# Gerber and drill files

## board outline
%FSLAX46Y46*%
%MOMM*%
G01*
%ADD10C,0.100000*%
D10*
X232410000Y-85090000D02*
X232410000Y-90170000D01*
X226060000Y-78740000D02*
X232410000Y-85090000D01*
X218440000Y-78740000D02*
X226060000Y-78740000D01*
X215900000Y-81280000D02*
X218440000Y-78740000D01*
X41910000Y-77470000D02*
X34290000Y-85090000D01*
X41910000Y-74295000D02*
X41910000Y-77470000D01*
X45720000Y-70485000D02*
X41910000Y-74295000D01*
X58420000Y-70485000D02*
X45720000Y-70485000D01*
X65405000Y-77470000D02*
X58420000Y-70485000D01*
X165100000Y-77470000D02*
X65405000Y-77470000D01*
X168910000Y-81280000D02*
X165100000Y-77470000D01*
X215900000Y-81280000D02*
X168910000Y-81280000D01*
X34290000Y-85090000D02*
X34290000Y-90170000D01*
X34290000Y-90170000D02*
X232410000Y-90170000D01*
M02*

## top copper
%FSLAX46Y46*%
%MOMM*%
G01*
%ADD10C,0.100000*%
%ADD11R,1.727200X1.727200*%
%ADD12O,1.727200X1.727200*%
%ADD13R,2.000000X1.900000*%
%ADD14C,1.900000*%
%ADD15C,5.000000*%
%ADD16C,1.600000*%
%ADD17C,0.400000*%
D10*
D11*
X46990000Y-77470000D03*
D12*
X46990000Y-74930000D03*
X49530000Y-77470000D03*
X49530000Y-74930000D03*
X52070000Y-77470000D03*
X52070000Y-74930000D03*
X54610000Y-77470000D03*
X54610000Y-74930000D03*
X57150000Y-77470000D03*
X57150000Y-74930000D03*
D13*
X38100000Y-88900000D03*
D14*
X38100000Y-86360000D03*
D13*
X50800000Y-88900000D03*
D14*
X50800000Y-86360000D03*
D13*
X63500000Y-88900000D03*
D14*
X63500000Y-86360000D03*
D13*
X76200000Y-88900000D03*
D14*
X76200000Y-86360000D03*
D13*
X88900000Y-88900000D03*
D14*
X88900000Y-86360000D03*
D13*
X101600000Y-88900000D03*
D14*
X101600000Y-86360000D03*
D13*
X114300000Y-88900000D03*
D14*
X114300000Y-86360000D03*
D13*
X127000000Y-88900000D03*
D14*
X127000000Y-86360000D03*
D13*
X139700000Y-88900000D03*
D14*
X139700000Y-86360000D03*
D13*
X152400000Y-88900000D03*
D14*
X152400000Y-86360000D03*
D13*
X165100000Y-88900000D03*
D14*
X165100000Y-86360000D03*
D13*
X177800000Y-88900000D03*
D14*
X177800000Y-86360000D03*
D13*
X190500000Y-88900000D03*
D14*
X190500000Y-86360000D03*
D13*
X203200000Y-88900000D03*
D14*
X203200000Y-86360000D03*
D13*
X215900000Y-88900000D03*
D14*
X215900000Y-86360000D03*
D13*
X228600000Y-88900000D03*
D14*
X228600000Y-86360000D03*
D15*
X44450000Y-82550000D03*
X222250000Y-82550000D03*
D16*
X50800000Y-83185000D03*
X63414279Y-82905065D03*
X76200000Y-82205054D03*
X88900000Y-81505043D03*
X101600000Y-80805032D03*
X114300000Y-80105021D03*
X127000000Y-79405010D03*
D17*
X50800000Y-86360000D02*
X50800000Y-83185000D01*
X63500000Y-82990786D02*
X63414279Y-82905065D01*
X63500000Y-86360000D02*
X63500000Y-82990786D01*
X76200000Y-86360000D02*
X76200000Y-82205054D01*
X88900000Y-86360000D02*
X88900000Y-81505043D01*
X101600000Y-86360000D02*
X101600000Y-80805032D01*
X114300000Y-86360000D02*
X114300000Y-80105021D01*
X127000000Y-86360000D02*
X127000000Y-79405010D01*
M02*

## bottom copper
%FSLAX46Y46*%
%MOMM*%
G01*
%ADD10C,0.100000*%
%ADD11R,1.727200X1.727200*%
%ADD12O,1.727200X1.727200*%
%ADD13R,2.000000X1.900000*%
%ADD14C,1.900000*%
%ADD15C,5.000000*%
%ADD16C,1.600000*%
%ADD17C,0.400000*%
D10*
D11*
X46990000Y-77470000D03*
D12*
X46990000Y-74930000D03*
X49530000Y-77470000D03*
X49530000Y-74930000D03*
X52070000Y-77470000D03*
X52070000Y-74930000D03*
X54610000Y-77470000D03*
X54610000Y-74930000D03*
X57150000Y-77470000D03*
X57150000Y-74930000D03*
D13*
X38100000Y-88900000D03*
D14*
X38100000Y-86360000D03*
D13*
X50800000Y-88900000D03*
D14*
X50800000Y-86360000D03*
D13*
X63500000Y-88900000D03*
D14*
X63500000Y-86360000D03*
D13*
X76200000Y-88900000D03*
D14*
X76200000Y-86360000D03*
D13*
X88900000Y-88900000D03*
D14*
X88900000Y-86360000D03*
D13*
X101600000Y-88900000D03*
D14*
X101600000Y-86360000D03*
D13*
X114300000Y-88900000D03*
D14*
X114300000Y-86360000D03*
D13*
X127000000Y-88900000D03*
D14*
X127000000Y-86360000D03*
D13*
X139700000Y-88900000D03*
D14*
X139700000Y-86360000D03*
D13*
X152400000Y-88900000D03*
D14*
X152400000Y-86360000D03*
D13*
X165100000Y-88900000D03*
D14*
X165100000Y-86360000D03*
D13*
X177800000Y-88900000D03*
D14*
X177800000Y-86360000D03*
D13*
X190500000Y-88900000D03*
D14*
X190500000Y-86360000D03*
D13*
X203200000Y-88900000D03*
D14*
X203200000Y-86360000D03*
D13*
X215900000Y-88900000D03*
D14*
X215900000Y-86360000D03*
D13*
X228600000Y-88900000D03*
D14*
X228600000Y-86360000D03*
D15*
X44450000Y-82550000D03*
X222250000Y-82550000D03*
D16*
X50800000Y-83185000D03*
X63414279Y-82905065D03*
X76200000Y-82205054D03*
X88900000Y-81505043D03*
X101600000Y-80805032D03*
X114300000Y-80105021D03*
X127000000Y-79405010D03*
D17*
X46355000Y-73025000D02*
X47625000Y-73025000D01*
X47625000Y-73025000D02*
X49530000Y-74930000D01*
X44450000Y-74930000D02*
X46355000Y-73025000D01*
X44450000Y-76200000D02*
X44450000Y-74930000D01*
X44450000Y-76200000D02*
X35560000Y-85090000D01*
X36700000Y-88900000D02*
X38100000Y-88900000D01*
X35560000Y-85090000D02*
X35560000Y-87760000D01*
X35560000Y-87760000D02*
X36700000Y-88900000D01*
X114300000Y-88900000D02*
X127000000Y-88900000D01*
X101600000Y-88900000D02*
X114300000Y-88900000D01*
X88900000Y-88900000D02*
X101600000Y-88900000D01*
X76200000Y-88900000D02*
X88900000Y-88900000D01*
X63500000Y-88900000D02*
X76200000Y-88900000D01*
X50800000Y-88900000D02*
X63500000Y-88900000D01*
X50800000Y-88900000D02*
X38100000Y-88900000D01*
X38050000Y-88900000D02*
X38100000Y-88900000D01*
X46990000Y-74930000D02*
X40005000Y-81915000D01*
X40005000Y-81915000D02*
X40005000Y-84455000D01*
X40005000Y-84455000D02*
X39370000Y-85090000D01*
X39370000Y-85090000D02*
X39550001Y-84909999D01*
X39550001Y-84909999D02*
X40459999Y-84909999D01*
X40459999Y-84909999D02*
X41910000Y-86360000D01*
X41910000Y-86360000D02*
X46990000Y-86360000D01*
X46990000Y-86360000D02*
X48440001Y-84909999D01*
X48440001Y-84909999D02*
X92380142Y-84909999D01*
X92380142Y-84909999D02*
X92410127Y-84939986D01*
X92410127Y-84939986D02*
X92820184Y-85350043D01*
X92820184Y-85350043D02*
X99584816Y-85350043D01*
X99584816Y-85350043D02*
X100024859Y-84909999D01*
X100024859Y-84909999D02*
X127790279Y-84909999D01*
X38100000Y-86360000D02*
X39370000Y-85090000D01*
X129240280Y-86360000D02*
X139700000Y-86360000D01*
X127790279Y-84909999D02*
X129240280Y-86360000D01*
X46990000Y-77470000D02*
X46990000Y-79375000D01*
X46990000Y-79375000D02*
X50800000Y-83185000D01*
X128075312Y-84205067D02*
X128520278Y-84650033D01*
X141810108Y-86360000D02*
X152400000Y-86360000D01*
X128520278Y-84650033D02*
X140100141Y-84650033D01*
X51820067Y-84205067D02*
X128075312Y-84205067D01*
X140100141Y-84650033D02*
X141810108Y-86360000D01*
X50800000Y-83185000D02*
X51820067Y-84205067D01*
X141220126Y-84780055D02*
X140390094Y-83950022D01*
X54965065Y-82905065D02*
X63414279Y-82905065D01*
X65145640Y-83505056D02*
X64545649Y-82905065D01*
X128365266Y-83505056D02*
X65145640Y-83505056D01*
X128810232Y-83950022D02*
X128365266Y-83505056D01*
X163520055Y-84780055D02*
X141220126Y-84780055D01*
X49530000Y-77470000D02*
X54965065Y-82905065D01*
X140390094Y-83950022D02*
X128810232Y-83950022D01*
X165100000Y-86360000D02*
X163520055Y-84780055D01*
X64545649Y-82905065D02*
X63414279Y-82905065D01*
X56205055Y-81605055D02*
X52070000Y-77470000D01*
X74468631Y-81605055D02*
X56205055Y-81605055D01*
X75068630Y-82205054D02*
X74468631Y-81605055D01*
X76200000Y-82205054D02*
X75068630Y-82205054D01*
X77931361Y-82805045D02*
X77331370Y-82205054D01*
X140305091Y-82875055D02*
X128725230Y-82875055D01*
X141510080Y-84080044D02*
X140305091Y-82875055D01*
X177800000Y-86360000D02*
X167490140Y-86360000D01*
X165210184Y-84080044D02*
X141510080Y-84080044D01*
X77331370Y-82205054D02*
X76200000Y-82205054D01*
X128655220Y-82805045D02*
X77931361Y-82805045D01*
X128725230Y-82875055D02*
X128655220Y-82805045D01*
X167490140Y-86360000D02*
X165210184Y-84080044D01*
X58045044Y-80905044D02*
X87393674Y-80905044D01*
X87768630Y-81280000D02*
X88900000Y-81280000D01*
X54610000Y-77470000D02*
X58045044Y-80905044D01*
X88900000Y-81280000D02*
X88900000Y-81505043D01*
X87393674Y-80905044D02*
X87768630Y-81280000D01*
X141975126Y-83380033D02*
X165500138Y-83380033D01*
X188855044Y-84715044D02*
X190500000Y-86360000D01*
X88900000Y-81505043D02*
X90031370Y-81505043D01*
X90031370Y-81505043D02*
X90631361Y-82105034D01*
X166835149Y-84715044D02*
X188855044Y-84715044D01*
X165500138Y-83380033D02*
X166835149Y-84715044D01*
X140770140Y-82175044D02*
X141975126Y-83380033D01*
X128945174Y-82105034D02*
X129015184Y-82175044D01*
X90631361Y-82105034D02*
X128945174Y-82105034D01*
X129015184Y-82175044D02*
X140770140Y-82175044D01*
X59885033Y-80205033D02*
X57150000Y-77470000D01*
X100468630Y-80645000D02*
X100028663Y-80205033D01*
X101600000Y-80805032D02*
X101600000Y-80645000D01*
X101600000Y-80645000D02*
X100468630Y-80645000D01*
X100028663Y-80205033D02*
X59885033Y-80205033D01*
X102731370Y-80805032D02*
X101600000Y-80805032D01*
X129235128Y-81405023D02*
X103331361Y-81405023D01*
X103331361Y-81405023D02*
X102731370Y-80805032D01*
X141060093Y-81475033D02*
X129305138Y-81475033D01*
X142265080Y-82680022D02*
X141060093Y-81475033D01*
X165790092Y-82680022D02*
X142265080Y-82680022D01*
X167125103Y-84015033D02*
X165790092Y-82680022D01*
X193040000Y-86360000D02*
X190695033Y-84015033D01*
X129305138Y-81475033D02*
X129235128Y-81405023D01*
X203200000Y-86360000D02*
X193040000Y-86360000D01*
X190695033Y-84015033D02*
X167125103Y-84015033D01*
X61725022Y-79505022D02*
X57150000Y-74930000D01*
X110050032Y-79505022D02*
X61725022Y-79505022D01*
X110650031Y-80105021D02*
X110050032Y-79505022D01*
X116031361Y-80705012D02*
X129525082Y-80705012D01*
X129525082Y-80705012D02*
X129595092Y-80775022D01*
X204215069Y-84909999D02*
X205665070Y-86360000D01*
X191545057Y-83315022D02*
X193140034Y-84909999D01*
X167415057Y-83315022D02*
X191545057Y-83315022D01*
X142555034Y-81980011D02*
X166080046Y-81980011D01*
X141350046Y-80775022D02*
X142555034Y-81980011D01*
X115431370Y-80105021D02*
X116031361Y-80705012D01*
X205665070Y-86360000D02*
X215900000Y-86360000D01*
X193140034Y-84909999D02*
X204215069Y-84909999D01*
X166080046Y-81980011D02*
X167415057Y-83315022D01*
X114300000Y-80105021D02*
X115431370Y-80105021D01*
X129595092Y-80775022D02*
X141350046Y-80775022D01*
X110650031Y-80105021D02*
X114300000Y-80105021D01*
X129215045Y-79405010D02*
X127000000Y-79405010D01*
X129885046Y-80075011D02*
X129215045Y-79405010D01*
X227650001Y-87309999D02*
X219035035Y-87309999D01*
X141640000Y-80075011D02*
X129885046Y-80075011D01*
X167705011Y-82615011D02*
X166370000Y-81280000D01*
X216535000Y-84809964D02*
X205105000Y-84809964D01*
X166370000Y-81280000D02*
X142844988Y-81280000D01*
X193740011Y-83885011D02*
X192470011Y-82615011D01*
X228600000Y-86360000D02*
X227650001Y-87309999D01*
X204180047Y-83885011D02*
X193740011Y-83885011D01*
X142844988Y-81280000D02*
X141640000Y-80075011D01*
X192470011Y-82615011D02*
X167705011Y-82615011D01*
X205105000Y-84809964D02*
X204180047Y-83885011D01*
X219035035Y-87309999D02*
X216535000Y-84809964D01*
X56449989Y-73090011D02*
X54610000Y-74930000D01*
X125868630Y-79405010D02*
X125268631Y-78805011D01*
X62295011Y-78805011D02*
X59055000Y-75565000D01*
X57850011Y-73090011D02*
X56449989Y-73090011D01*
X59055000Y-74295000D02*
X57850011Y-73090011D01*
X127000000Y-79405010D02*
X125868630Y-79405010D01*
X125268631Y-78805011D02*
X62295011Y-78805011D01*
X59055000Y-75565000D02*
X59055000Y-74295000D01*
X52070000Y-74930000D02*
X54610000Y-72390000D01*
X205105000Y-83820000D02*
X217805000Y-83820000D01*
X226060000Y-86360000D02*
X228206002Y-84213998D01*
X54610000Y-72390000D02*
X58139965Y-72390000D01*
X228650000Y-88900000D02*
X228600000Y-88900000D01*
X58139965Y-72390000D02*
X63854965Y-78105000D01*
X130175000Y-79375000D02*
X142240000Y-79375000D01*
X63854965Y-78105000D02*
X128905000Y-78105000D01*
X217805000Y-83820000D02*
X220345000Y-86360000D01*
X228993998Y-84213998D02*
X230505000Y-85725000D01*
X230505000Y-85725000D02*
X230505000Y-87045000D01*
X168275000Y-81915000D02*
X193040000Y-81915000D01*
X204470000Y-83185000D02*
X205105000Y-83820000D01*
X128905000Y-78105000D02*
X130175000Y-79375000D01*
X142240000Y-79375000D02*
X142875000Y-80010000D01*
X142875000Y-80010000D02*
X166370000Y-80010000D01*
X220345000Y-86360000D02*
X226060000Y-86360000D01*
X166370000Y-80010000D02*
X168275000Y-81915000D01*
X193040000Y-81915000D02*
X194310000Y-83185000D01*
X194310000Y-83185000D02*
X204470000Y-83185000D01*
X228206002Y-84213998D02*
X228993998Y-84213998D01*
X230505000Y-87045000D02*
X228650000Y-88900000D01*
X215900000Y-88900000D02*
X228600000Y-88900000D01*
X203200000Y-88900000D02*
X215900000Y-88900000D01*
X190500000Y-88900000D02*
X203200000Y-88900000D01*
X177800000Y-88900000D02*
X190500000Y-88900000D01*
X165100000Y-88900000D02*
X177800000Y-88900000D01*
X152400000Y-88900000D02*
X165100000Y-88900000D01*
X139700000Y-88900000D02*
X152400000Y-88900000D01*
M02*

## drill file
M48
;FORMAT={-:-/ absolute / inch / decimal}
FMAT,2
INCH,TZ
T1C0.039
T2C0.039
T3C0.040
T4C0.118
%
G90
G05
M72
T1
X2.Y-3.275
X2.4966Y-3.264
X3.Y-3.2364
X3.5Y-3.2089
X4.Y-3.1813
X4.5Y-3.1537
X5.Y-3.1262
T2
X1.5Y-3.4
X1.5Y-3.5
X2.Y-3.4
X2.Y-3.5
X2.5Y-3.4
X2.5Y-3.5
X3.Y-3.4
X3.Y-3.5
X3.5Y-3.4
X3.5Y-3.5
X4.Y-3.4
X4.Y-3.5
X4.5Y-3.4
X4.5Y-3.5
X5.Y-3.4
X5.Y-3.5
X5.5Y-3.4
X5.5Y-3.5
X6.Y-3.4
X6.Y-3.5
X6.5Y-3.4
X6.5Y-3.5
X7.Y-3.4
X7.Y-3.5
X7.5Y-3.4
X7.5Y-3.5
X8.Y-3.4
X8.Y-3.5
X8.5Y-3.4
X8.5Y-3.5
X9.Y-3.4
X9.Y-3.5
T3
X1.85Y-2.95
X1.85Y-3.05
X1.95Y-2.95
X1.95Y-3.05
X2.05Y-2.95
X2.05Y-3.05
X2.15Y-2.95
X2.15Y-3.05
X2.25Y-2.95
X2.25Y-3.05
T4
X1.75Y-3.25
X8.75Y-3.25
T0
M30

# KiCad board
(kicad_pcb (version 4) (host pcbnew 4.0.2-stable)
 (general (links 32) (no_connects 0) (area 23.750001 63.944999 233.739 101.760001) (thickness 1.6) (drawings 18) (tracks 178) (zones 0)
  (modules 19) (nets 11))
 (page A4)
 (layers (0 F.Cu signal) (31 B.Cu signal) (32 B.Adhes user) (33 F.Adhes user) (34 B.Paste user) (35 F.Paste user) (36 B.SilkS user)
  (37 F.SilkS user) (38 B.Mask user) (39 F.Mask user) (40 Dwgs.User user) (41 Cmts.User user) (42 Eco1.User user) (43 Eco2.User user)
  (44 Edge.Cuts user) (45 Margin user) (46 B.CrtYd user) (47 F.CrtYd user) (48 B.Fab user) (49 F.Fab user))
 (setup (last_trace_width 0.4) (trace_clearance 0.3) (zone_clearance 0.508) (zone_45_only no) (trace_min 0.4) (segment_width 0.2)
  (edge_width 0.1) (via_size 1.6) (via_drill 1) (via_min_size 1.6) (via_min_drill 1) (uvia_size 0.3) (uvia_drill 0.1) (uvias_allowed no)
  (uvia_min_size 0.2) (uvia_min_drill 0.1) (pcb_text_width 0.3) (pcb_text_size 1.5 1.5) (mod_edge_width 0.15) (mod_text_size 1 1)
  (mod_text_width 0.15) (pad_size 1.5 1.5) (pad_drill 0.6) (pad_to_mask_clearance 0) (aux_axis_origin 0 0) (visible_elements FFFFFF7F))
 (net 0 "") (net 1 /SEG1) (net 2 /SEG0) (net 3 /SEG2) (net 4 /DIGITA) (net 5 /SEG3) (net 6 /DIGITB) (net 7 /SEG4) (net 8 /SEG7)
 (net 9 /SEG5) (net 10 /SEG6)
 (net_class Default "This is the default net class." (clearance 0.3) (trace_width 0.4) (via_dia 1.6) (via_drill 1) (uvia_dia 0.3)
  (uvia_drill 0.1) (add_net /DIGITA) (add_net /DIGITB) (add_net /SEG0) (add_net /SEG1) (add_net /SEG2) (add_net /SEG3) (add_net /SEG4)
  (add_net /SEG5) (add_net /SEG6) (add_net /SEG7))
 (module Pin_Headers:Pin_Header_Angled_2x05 (layer F.Cu) (at 46.99 77.47 90)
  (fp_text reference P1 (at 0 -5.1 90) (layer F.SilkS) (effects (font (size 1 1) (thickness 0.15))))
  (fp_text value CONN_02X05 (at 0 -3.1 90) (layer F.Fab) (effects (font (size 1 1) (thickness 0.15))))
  (pad 1 thru_hole rect (at 0 0 90) (size 1.7272 1.7272) (drill 1.016) (layers *.Cu *.Mask F.SilkS) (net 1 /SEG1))
  (pad 2 thru_hole oval (at 2.54 0 90) (size 1.7272 1.7272) (drill 1.016) (layers *.Cu *.Mask F.SilkS) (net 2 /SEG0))
  (pad 3 thru_hole oval (at 0 2.54 90) (size 1.7272 1.7272) (drill 1.016) (layers *.Cu *.Mask F.SilkS) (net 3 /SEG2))
  (pad 4 thru_hole oval (at 2.54 2.54 90) (size 1.7272 1.7272) (drill 1.016) (layers *.Cu *.Mask F.SilkS) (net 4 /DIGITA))
  (pad 5 thru_hole oval (at 0 5.08 90) (size 1.7272 1.7272) (drill 1.016) (layers *.Cu *.Mask F.SilkS) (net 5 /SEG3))
  (pad 6 thru_hole oval (at 2.54 5.08 90) (size 1.7272 1.7272) (drill 1.016) (layers *.Cu *.Mask F.SilkS) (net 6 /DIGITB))
  (pad 7 thru_hole oval (at 0 7.62 90) (size 1.7272 1.7272) (drill 1.016) (layers *.Cu *.Mask F.SilkS) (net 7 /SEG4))
  (pad 8 thru_hole oval (at 2.54 7.62 90) (size 1.7272 1.7272) (drill 1.016) (layers *.Cu *.Mask F.SilkS) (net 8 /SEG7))
  (pad 9 thru_hole oval (at 0 10.16 90) (size 1.7272 1.7272) (drill 1.016) (layers *.Cu *.Mask F.SilkS) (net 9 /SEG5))
  (pad 10 thru_hole oval (at 2.54 10.16 90) (size 1.7272 1.7272) (drill 1.016) (layers *.Cu *.Mask F.SilkS) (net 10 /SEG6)))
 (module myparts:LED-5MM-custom (layer F.Cu) (at 38.1 88.9 90)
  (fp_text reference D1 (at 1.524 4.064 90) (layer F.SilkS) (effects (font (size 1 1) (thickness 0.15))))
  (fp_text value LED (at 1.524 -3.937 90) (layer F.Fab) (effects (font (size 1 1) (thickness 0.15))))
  (pad 1 thru_hole rect (at 0 0 180) (size 2 1.9) (drill 1.00076) (layers *.Cu *.Mask F.SilkS) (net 4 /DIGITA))
  (pad 2 thru_hole circle (at 2.54 0 90) (size 1.9 1.9) (drill 1.00076) (layers *.Cu *.Mask F.SilkS) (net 2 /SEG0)))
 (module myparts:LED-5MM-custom (layer F.Cu) (at 50.8 88.9 90)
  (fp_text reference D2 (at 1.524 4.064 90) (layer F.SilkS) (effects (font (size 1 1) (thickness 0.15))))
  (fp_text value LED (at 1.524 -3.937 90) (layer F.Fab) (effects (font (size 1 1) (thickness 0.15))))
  (pad 1 thru_hole rect (at 0 0 180) (size 2 1.9) (drill 1.00076) (layers *.Cu *.Mask F.SilkS) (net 4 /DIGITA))
  (pad 2 thru_hole circle (at 2.54 0 90) (size 1.9 1.9) (drill 1.00076) (layers *.Cu *.Mask F.SilkS) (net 1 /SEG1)))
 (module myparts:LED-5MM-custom (layer F.Cu) (at 63.5 88.9 90)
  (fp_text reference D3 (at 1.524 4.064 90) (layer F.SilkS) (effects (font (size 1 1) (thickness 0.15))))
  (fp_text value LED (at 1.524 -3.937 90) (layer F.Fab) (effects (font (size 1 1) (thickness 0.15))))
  (pad 1 thru_hole rect (at 0 0 180) (size 2 1.9) (drill 1.00076) (layers *.Cu *.Mask F.SilkS) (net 4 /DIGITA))
  (pad 2 thru_hole circle (at 2.54 0 90) (size 1.9 1.9) (drill 1.00076) (layers *.Cu *.Mask F.SilkS) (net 3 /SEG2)))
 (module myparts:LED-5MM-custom (layer F.Cu) (at 76.2 88.9 90)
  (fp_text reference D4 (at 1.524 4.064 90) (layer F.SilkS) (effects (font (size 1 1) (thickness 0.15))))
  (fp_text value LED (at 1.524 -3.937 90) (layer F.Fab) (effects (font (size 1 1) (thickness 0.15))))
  (pad 1 thru_hole rect (at 0 0 180) (size 2 1.9) (drill 1.00076) (layers *.Cu *.Mask F.SilkS) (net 4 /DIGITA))
  (pad 2 thru_hole circle (at 2.54 0 90) (size 1.9 1.9) (drill 1.00076) (layers *.Cu *.Mask F.SilkS) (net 5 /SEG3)))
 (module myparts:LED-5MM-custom (layer F.Cu) (at 88.9 88.9 90)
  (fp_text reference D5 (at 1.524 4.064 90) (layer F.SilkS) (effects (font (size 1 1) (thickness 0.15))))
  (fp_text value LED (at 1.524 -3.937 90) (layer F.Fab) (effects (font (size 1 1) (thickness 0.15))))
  (pad 1 thru_hole rect (at 0 0 180) (size 2 1.9) (drill 1.00076) (layers *.Cu *.Mask F.SilkS) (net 4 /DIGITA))
  (pad 2 thru_hole circle (at 2.54 0 90) (size 1.9 1.9) (drill 1.00076) (layers *.Cu *.Mask F.SilkS) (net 7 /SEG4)))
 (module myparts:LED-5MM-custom (layer F.Cu) (at 101.6 88.9 90)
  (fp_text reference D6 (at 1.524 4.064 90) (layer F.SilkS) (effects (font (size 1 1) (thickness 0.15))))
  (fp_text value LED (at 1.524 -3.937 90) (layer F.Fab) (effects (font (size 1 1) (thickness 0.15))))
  (pad 1 thru_hole rect (at 0 0 180) (size 2 1.9) (drill 1.00076) (layers *.Cu *.Mask F.SilkS) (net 4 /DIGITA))
  (pad 2 thru_hole circle (at 2.54 0 90) (size 1.9 1.9) (drill 1.00076) (layers *.Cu *.Mask F.SilkS) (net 9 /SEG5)))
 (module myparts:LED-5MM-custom (layer F.Cu) (at 114.3 88.9 90)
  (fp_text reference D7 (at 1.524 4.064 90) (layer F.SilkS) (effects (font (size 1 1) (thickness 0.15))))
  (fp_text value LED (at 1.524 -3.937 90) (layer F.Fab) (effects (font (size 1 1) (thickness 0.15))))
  (pad 1 thru_hole rect (at 0 0 180) (size 2 1.9) (drill 1.00076) (layers *.Cu *.Mask F.SilkS) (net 4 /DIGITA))
  (pad 2 thru_hole circle (at 2.54 0 90) (size 1.9 1.9) (drill 1.00076) (layers *.Cu *.Mask F.SilkS) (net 10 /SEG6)))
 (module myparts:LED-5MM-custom (layer F.Cu) (at 127 88.9 90)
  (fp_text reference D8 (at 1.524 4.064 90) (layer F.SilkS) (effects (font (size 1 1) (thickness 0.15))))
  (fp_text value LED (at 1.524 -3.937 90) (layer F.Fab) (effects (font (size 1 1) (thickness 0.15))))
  (pad 1 thru_hole rect (at 0 0 180) (size 2 1.9) (drill 1.00076) (layers *.Cu *.Mask F.SilkS) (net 4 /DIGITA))
  (pad 2 thru_hole circle (at 2.54 0 90) (size 1.9 1.9) (drill 1.00076) (layers *.Cu *.Mask F.SilkS) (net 8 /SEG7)))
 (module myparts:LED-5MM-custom (layer F.Cu) (at 139.7 88.9 90)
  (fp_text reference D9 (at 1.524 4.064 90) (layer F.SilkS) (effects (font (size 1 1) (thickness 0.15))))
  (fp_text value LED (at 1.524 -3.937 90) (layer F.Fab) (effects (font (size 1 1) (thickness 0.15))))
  (pad 1 thru_hole rect (at 0 0 180) (size 2 1.9) (drill 1.00076) (layers *.Cu *.Mask F.SilkS) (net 6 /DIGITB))
  (pad 2 thru_hole circle (at 2.54 0 90) (size 1.9 1.9) (drill 1.00076) (layers *.Cu *.Mask F.SilkS) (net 2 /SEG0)))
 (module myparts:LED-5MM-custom (layer F.Cu) (at 152.4 88.9 90)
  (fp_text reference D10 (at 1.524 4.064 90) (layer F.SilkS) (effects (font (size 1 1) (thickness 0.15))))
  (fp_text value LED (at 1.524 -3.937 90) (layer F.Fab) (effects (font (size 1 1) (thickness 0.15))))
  (pad 1 thru_hole rect (at 0 0 180) (size 2 1.9) (drill 1.00076) (layers *.Cu *.Mask F.SilkS) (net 6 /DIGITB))
  (pad 2 thru_hole circle (at 2.54 0 90) (size 1.9 1.9) (drill 1.00076) (layers *.Cu *.Mask F.SilkS) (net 1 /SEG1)))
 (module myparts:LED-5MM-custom (layer F.Cu) (at 165.1 88.9 90)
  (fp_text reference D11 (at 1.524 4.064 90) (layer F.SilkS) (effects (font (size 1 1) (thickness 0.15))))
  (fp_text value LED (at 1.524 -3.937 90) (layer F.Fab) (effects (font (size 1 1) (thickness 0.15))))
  (pad 1 thru_hole rect (at 0 0 180) (size 2 1.9) (drill 1.00076) (layers *.Cu *.Mask F.SilkS) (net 6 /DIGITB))
  (pad 2 thru_hole circle (at 2.54 0 90) (size 1.9 1.9) (drill 1.00076) (layers *.Cu *.Mask F.SilkS) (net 3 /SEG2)))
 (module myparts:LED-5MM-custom (layer F.Cu) (at 177.8 88.9 90)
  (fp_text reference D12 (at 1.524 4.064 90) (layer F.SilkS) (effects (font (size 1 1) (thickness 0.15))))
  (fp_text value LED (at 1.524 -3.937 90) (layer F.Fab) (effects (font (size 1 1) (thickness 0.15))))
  (pad 1 thru_hole rect (at 0 0 180) (size 2 1.9) (drill 1.00076) (layers *.Cu *.Mask F.SilkS) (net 6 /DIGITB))
  (pad 2 thru_hole circle (at 2.54 0 90) (size 1.9 1.9) (drill 1.00076) (layers *.Cu *.Mask F.SilkS) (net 5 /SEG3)))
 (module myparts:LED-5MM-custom (layer F.Cu) (at 190.5 88.9 90)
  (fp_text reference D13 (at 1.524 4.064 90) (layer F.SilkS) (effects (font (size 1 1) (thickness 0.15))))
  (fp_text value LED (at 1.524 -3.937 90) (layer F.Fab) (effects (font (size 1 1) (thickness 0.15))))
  (pad 1 thru_hole rect (at 0 0 180) (size 2 1.9) (drill 1.00076) (layers *.Cu *.Mask F.SilkS) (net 6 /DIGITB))
  (pad 2 thru_hole circle (at 2.54 0 90) (size 1.9 1.9) (drill 1.00076) (layers *.Cu *.Mask F.SilkS) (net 7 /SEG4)))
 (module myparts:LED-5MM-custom (layer F.Cu) (at 203.2 88.9 90)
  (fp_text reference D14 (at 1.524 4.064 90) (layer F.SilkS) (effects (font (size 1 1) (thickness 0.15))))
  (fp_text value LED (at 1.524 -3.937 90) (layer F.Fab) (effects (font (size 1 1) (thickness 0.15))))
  (pad 1 thru_hole rect (at 0 0 180) (size 2 1.9) (drill 1.00076) (layers *.Cu *.Mask F.SilkS) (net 6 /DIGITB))
  (pad 2 thru_hole circle (at 2.54 0 90) (size 1.9 1.9) (drill 1.00076) (layers *.Cu *.Mask F.SilkS) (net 9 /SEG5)))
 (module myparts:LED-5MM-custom (layer F.Cu) (at 215.9 88.9 90)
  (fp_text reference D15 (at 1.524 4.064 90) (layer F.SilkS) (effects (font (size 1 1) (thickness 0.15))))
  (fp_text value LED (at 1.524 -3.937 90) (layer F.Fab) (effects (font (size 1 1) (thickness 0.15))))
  (pad 1 thru_hole rect (at 0 0 180) (size 2 1.9) (drill 1.00076) (layers *.Cu *.Mask F.SilkS) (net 6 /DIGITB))
  (pad 2 thru_hole circle (at 2.54 0 90) (size 1.9 1.9) (drill 1.00076) (layers *.Cu *.Mask F.SilkS) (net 10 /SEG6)))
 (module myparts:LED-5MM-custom (layer F.Cu) (at 228.6 88.9 90)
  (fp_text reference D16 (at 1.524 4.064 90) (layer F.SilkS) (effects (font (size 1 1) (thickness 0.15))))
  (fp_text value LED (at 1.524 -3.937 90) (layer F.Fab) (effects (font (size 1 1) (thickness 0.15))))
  (pad 1 thru_hole rect (at 0 0 180) (size 2 1.9) (drill 1.00076) (layers *.Cu *.Mask F.SilkS) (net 6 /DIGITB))
  (pad 2 thru_hole circle (at 2.54 0 90) (size 1.9 1.9) (drill 1.00076) (layers *.Cu *.Mask F.SilkS) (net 8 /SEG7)))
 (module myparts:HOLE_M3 (layer F.Cu) (at 44.45 82.55)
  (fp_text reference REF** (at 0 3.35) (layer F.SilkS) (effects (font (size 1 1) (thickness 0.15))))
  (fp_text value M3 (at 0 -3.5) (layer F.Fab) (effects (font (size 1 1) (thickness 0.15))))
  (pad 1 thru_hole circle (at 0 0) (size 5 5) (drill 3) (layers *.Cu *.Mask F.SilkS)))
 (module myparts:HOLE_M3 (layer F.Cu) (at 222.25 82.55)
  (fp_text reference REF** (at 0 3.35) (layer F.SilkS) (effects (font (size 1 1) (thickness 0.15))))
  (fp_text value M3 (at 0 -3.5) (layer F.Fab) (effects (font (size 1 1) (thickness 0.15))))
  (pad 1 thru_hole circle (at 0 0) (size 5 5) (drill 3) (layers *.Cu *.Mask F.SilkS)))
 (gr_line (start 232.41 85.09) (end 232.41 90.17) (layer Edge.Cuts) (width 0.1))
 (gr_line (start 226.06 78.74) (end 232.41 85.09) (layer Edge.Cuts) (width 0.1))
 (gr_line (start 218.44 78.74) (end 226.06 78.74) (layer Edge.Cuts) (width 0.1))
 (gr_line (start 215.9 81.28) (end 218.44 78.74) (layer Edge.Cuts) (width 0.1))
 (gr_line (start 41.91 77.47) (end 34.29 85.09) (layer Edge.Cuts) (width 0.1))
 (gr_line (start 41.91 74.295) (end 41.91 77.47) (layer Edge.Cuts) (width 0.1))
 (gr_line (start 45.72 70.485) (end 41.91 74.295) (layer Edge.Cuts) (width 0.1))
 (gr_line (start 58.42 70.485) (end 45.72 70.485) (layer Edge.Cuts) (width 0.1))
 (gr_line (start 65.405 77.47) (end 58.42 70.485) (layer Edge.Cuts) (width 0.1))
 (gr_line (start 165.1 77.47) (end 65.405 77.47) (layer Edge.Cuts) (width 0.1))
 (gr_line (start 168.91 81.28) (end 165.1 77.47) (layer Edge.Cuts) (width 0.1))
 (gr_line (start 215.9 81.28) (end 168.91 81.28) (layer Edge.Cuts) (width 0.1))
 (gr_line (start 34.29 85.09) (end 34.29 90.17) (layer Edge.Cuts) (width 0.1))
 (gr_line (start 34.29 90.17) (end 232.41 90.17) (layer Edge.Cuts) (width 0.1))
 (segment (start 46.355 73.025) (end 47.625 73.025) (width 0.4) (layer B.Cu) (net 4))
 (segment (start 47.625 73.025) (end 49.53 74.93) (width 0.4) (layer B.Cu) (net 4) (status 20))
 (segment (start 44.45 74.93) (end 46.355 73.025) (width 0.4) (layer B.Cu) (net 4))
 (segment (start 44.45 76.2) (end 44.45 74.93) (width 0.4) (layer B.Cu) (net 4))
 (segment (start 44.45 76.2) (end 35.56 85.09) (width 0.4) (layer B.Cu) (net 4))
 (segment (start 36.7 88.9) (end 38.1 88.9) (width 0.4) (layer B.Cu) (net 4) (status 20))
 (segment (start 35.56 85.09) (end 35.56 87.76) (width 0.4) (layer B.Cu) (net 4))
 (segment (start 35.56 87.76) (end 36.7 88.9) (width 0.4) (layer B.Cu) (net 4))
 (segment (start 114.3 88.9) (end 127 88.9) (width 0.4) (layer B.Cu) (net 4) (status 30))
 (segment (start 101.6 88.9) (end 114.3 88.9) (width 0.4) (layer B.Cu) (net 4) (status 30))
 (segment (start 88.9 88.9) (end 101.6 88.9) (width 0.4) (layer B.Cu) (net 4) (status 30))
 (segment (start 76.2 88.9) (end 88.9 88.9) (width 0.4) (layer B.Cu) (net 4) (status 30))
 (segment (start 63.5 88.9) (end 76.2 88.9) (width 0.4) (layer B.Cu) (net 4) (status 30))
 (segment (start 50.8 88.9) (end 63.5 88.9) (width 0.4) (layer B.Cu) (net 4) (status 30))
 (segment (start 50.8 88.9) (end 38.1 88.9) (width 0.4) (layer B.Cu) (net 4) (status 30))
 (segment (start 38.05 88.9) (end 38.1 88.9) (width 0.4) (layer B.Cu) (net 4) (status 30))
 (segment (start 46.99 74.93) (end 40.005 81.915) (width 0.4) (layer B.Cu) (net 2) (status 10))
 (segment (start 40.005 81.915) (end 40.005 84.455) (width 0.4) (layer B.Cu) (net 2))
 (segment (start 40.005 84.455) (end 39.37 85.09) (width 0.4) (layer B.Cu) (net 2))
 (segment (start 39.37 85.09) (end 39.550001 84.909999) (width 0.4) (layer B.Cu) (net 2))
 (segment (start 39.550001 84.909999) (end 40.459999 84.909999) (width 0.4) (layer B.Cu) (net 2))
 (segment (start 40.459999 84.909999) (end 41.91 86.36) (width 0.4) (layer B.Cu) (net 2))
 (segment (start 41.91 86.36) (end 46.99 86.36) (width 0.4) (layer B.Cu) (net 2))
 (segment (start 46.99 86.36) (end 48.440001 84.909999) (width 0.4) (layer B.Cu) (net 2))
 (segment (start 48.440001 84.909999) (end 92.380142 84.909999) (width 0.4) (layer B.Cu) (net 2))
 (segment (start 92.380142 84.909999) (end 92.410127 84.939986) (width 0.4) (layer B.Cu) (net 2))
 (segment (start 92.410127 84.939986) (end 92.820184 85.350043) (width 0.4) (layer B.Cu) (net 2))
 (segment (start 92.820184 85.350043) (end 99.584816 85.350043) (width 0.4) (layer B.Cu) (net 2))
 (segment (start 99.584816 85.350043) (end 100.024859 84.909999) (width 0.4) (layer B.Cu) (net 2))
 (segment (start 100.024859 84.909999) (end 127.790279 84.909999) (width 0.4) (layer B.Cu) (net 2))
 (segment (start 38.1 86.36) (end 39.37 85.09) (width 0.4) (layer B.Cu) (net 2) (status 10))
 (segment (start 129.24028 86.36) (end 139.7 86.36) (width 0.4) (layer B.Cu) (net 2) (status 20))
 (segment (start 127.790279 84.909999) (end 129.24028 86.36) (width 0.4) (layer B.Cu) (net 2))
 (segment (start 46.99 77.47) (end 46.99 79.375) (width 0.4) (layer B.Cu) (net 1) (status 10))
 (segment (start 46.99 79.375) (end 50.8 83.185) (width 0.4) (layer B.Cu) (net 1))
 (segment (start 128.075312 84.205067) (end 128.520278 84.650033) (width 0.4) (layer B.Cu) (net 1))
 (segment (start 141.810108 86.36) (end 152.4 86.36) (width 0.4) (layer B.Cu) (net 1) (status 20))
 (segment (start 128.520278 84.650033) (end 140.100141 84.650033) (width 0.4) (layer B.Cu) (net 1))
 (segment (start 51.820067 84.205067) (end 128.075312 84.205067) (width 0.4) (layer B.Cu) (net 1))
 (segment (start 140.100141 84.650033) (end 141.810108 86.36) (width 0.4) (layer B.Cu) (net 1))
 (segment (start 50.8 83.185) (end 51.820067 84.205067) (width 0.4) (layer B.Cu) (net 1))
 (segment (start 50.8 86.36) (end 50.8 83.185) (width 0.4) (layer F.Cu) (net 1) (status 10))
 (via (at 50.8 83.185) (size 1.6) (drill 1) (layers F.Cu B.Cu) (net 1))
 (segment (start 141.220126 84.780055) (end 140.390094 83.950022) (width 0.4) (layer B.Cu) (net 3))
 (segment (start 54.965065 82.905065) (end 63.414279 82.905065) (width 0.4) (layer B.Cu) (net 3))
 (segment (start 65.14564 83.505056) (end 64.545649 82.905065) (width 0.4) (layer B.Cu) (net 3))
 (segment (start 128.365266 83.505056) (end 65.14564 83.505056) (width 0.4) (layer B.Cu) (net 3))
 (segment (start 128.810232 83.950022) (end 128.365266 83.505056) (width 0.4) (layer B.Cu) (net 3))
 (segment (start 163.520055 84.780055) (end 141.220126 84.780055) (width 0.4) (layer B.Cu) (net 3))
 (segment (start 49.53 77.47) (end 54.965065 82.905065) (width 0.4) (layer B.Cu) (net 3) (status 10))
 (segment (start 63.5 82.990786) (end 63.414279 82.905065) (width 0.4) (layer F.Cu) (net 3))
 (segment (start 140.390094 83.950022) (end 128.810232 83.950022) (width 0.4) (layer B.Cu) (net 3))
 (segment (start 165.1 86.36) (end 163.520055 84.780055) (width 0.4) (layer B.Cu) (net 3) (status 10))
 (segment (start 63.5 86.36) (end 63.5 82.990786) (width 0.4) (layer F.Cu) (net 3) (status 10))
 (via (at 63.414279 82.905065) (size 1.6) (drill 1) (layers F.Cu B.Cu) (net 3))
 (segment (start 64.545649 82.905065) (end 63.414279 82.905065) (width 0.4) (layer B.Cu) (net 3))
 (segment (start 56.205055 81.605055) (end 52.07 77.47) (width 0.4) (layer B.Cu) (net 5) (status 20))
 (segment (start 74.468631 81.605055) (end 56.205055 81.605055) (width 0.4) (layer B.Cu) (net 5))
 (segment (start 75.06863 82.205054) (end 74.468631 81.605055) (width 0.4) (layer B.Cu) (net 5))
 (segment (start 76.2 82.205054) (end 75.06863 82.205054) (width 0.4) (layer B.Cu) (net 5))
 (segment (start 77.931361 82.805045) (end 77.33137 82.205054) (width 0.4) (layer B.Cu) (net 5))
 (segment (start 140.305091 82.875055) (end 128.72523 82.875055) (width 0.4) (layer B.Cu) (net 5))
 (segment (start 141.51008 84.080044) (end 140.305091 82.875055) (width 0.4) (layer B.Cu) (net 5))
 (segment (start 177.8 86.36) (end 167.49014 86.36) (width 0.4) (layer B.Cu) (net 5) (status 10))
 (segment (start 165.210184 84.080044) (end 141.51008 84.080044) (width 0.4) (layer B.Cu) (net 5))
 (segment (start 77.33137 82.205054) (end 76.2 82.205054) (width 0.4) (layer B.Cu) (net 5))
 (segment (start 128.65522 82.805045) (end 77.931361 82.805045) (width 0.4) (layer B.Cu) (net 5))
 (segment (start 128.72523 82.875055) (end 128.65522 82.805045) (width 0.4) (layer B.Cu) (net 5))
 (segment (start 167.49014 86.36) (end 165.210184 84.080044) (width 0.4) (layer B.Cu) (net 5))
 (segment (start 76.2 86.36) (end 76.2 82.205054) (width 0.4) (layer F.Cu) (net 5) (status 10))
 (via (at 76.2 82.205054) (size 1.6) (drill 1) (layers F.Cu B.Cu) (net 5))
 (segment (start 58.045044 80.905044) (end 87.393674 80.905044) (width 0.4) (layer B.Cu) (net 7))
 (segment (start 87.76863 81.28) (end 88.9 81.28) (width 0.4) (layer B.Cu) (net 7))
 (segment (start 54.61 77.47) (end 58.045044 80.905044) (width 0.4) (layer B.Cu) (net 7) (status 10))
 (segment (start 88.9 81.28) (end 88.9 81.505043) (width 0.4) (layer B.Cu) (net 7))
 (segment (start 87.393674 80.905044) (end 87.76863 81.28) (width 0.4) (layer B.Cu) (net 7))
 (segment (start 141.975126 83.380033) (end 165.500138 83.380033) (width 0.4) (layer B.Cu) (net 7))
 (segment (start 188.855044 84.715044) (end 190.5 86.36) (width 0.4) (layer B.Cu) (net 7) (status 20))
 (segment (start 88.9 81.505043) (end 90.03137 81.505043) (width 0.4) (layer B.Cu) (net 7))
 (segment (start 90.03137 81.505043) (end 90.631361 82.105034) (width 0.4) (layer B.Cu) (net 7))
 (segment (start 166.835149 84.715044) (end 188.855044 84.715044) (width 0.4) (layer B.Cu) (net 7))
 (segment (start 165.500138 83.380033) (end 166.835149 84.715044) (width 0.4) (layer B.Cu) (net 7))
 (segment (start 140.77014 82.175044) (end 141.975126 83.380033) (width 0.4) (layer B.Cu) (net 7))
 (segment (start 128.945174 82.105034) (end 129.015184 82.175044) (width 0.4) (layer B.Cu) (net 7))
 (segment (start 90.631361 82.105034) (end 128.945174 82.105034) (width 0.4) (layer B.Cu) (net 7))
 (segment (start 129.015184 82.175044) (end 140.77014 82.175044) (width 0.4) (layer B.Cu) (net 7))
 (segment (start 88.9 86.36) (end 88.9 81.505043) (width 0.4) (layer F.Cu) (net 7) (status 10))
 (via (at 88.9 81.505043) (size 1.6) (drill 1) (layers F.Cu B.Cu) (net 7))
 (segment (start 59.885033 80.205033) (end 57.15 77.47) (width 0.4) (layer B.Cu) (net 9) (status 20))
 (segment (start 100.46863 80.645) (end 100.028663 80.205033) (width 0.4) (layer B.Cu) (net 9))
 (segment (start 101.6 80.805032) (end 101.6 80.645) (width 0.4) (layer B.Cu) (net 9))
 (segment (start 101.6 80.645) (end 100.46863 80.645) (width 0.4) (layer B.Cu) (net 9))
 (segment (start 100.028663 80.205033) (end 59.885033 80.205033) (width 0.4) (layer B.Cu) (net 9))
 (segment (start 102.73137 80.805032) (end 101.6 80.805032) (width 0.4) (layer B.Cu) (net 9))
 (segment (start 129.235128 81.405023) (end 103.331361 81.405023) (width 0.4) (layer B.Cu) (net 9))
 (segment (start 103.331361 81.405023) (end 102.73137 80.805032) (width 0.4) (layer B.Cu) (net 9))
 (segment (start 141.060093 81.475033) (end 129.305138 81.475033) (width 0.4) (layer B.Cu) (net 9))
 (segment (start 142.26508 82.680022) (end 141.060093 81.475033) (width 0.4) (layer B.Cu) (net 9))
 (segment (start 165.790092 82.680022) (end 142.26508 82.680022) (width 0.4) (layer B.Cu) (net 9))
 (segment (start 167.125103 84.015033) (end 165.790092 82.680022) (width 0.4) (layer B.Cu) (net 9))
 (segment (start 193.04 86.36) (end 190.695033 84.015033) (width 0.4) (layer B.Cu) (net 9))
 (segment (start 129.305138 81.475033) (end 129.235128 81.405023) (width 0.4) (layer B.Cu) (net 9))
 (segment (start 203.2 86.36) (end 193.04 86.36) (width 0.4) (layer B.Cu) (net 9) (status 10))
 (segment (start 190.695033 84.015033) (end 167.125103 84.015033) (width 0.4) (layer B.Cu) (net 9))
 (segment (start 101.6 86.36) (end 101.6 80.805032) (width 0.4) (layer F.Cu) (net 9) (status 10))
 (via (at 101.6 80.805032) (size 1.6) (drill 1) (layers F.Cu B.Cu) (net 9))
 (segment (start 61.725022 79.505022) (end 57.15 74.93) (width 0.4) (layer B.Cu) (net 10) (status 20))
 (segment (start 110.050032 79.505022) (end 61.725022 79.505022) (width 0.4) (layer B.Cu) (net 10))
 (segment (start 110.650031 80.105021) (end 110.050032 79.505022) (width 0.4) (layer B.Cu) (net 10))
 (segment (start 116.031361 80.705012) (end 129.525082 80.705012) (width 0.4) (layer B.Cu) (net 10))
 (segment (start 129.525082 80.705012) (end 129.595092 80.775022) (width 0.4) (layer B.Cu) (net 10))
 (segment (start 204.215069 84.909999) (end 205.66507 86.36) (width 0.4) (layer B.Cu) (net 10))
 (segment (start 191.545057 83.315022) (end 193.140034 84.909999) (width 0.4) (layer B.Cu) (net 10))
 (segment (start 167.415057 83.315022) (end 191.545057 83.315022) (width 0.4) (layer B.Cu) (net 10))
 (segment (start 142.555034 81.980011) (end 166.080046 81.980011) (width 0.4) (layer B.Cu) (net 10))
 (segment (start 141.350046 80.775022) (end 142.555034 81.980011) (width 0.4) (layer B.Cu) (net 10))
 (segment (start 115.43137 80.105021) (end 116.031361 80.705012) (width 0.4) (layer B.Cu) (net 10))
 (segment (start 205.66507 86.36) (end 215.9 86.36) (width 0.4) (layer B.Cu) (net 10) (status 20))
 (segment (start 193.140034 84.909999) (end 204.215069 84.909999) (width 0.4) (layer B.Cu) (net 10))
 (segment (start 166.080046 81.980011) (end 167.415057 83.315022) (width 0.4) (layer B.Cu) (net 10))
 (segment (start 114.3 80.105021) (end 115.43137 80.105021) (width 0.4) (layer B.Cu) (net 10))
 (segment (start 129.595092 80.775022) (end 141.350046 80.775022) (width 0.4) (layer B.Cu) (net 10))
 (segment (start 110.650031 80.105021) (end 114.3 80.105021) (width 0.4) (layer B.Cu) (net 10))
 (segment (start 114.3 86.36) (end 114.3 80.105021) (width 0.4) (layer F.Cu) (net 10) (status 10))
 (via (at 114.3 80.105021) (size 1.6) (drill 1) (layers F.Cu B.Cu) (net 10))
 (segment (start 129.215045 79.40501) (end 127 79.40501) (width 0.4) (layer B.Cu) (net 8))
 (segment (start 129.885046 80.075011) (end 129.215045 79.40501) (width 0.4) (layer B.Cu) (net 8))
 (segment (start 227.650001 87.309999) (end 219.035035 87.309999) (width 0.4) (layer B.Cu) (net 8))
 (segment (start 141.64 80.075011) (end 129.885046 80.075011) (width 0.4) (layer B.Cu) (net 8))
 (segment (start 167.705011 82.615011) (end 166.37 81.28) (width 0.4) (layer B.Cu) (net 8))
 (segment (start 216.535 84.809964) (end 205.105 84.809964) (width 0.4) (layer B.Cu) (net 8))
 (segment (start 166.37 81.28) (end 142.844988 81.28) (width 0.4) (layer B.Cu) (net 8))
 (segment (start 193.740011 83.885011) (end 192.470011 82.615011) (width 0.4) (layer B.Cu) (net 8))
 (segment (start 228.6 86.36) (end 227.650001 87.309999) (width 0.4) (layer B.Cu) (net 8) (status 10))
 (segment (start 204.180047 83.885011) (end 193.740011 83.885011) (width 0.4) (layer B.Cu) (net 8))
 (segment (start 142.844988 81.28) (end 141.64 80.075011) (width 0.4) (layer B.Cu) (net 8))
 (segment (start 192.470011 82.615011) (end 167.705011 82.615011) (width 0.4) (layer B.Cu) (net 8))
 (segment (start 205.105 84.809964) (end 204.180047 83.885011) (width 0.4) (layer B.Cu) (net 8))
 (segment (start 219.035035 87.309999) (end 216.535 84.809964) (width 0.4) (layer B.Cu) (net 8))
 (segment (start 56.449989 73.090011) (end 54.61 74.93) (width 0.4) (layer B.Cu) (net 8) (status 20))
 (segment (start 125.86863 79.40501) (end 125.268631 78.805011) (width 0.4) (layer B.Cu) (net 8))
 (segment (start 62.295011 78.805011) (end 59.055 75.565) (width 0.4) (layer B.Cu) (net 8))
 (segment (start 57.850011 73.090011) (end 56.449989 73.090011) (width 0.4) (layer B.Cu) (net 8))
 (segment (start 59.055 74.295) (end 57.850011 73.090011) (width 0.4) (layer B.Cu) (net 8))
 (segment (start 127 79.40501) (end 125.86863 79.40501) (width 0.4) (layer B.Cu) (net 8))
 (segment (start 125.268631 78.805011) (end 62.295011 78.805011) (width 0.4) (layer B.Cu) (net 8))
 (segment (start 59.055 75.565) (end 59.055 74.295) (width 0.4) (layer B.Cu) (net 8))
 (via (at 127 79.40501) (size 1.6) (drill 1) (layers F.Cu B.Cu) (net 8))
 (segment (start 127 86.36) (end 127 79.40501) (width 0.4) (layer F.Cu) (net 8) (status 10))
 (segment (start 52.07 74.93) (end 54.61 72.39) (width 0.4) (layer B.Cu) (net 6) (status 10))
 (segment (start 205.105 83.82) (end 217.805 83.82) (width 0.4) (layer B.Cu) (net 6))
 (segment (start 226.06 86.36) (end 228.206002 84.213998) (width 0.4) (layer B.Cu) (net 6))
 (segment (start 54.61 72.39) (end 58.139965 72.39) (width 0.4) (layer B.Cu) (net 6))
 (segment (start 228.65 88.9) (end 228.6 88.9) (width 0.4) (layer B.Cu) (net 6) (status 30))
 (segment (start 58.139965 72.39) (end 63.854965 78.105) (width 0.4) (layer B.Cu) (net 6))
 (segment (start 130.175 79.375) (end 142.24 79.375) (width 0.4) (layer B.Cu) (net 6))
 (segment (start 63.854965 78.105) (end 128.905 78.105) (width 0.4) (layer B.Cu) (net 6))
 (segment (start 217.805 83.82) (end 220.345 86.36) (width 0.4) (layer B.Cu) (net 6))
 (segment (start 228.993998 84.213998) (end 230.505 85.725) (width 0.4) (layer B.Cu) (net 6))
 (segment (start 230.505 85.725) (end 230.505 87.045) (width 0.4) (layer B.Cu) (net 6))
 (segment (start 168.275 81.915) (end 193.04 81.915) (width 0.4) (layer B.Cu) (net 6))
 (segment (start 204.47 83.185) (end 205.105 83.82) (width 0.4) (layer B.Cu) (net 6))
 (segment (start 128.905 78.105) (end 130.175 79.375) (width 0.4) (layer B.Cu) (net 6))
 (segment (start 142.24 79.375) (end 142.875 80.01) (width 0.4) (layer B.Cu) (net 6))
 (segment (start 142.875 80.01) (end 166.37 80.01) (width 0.4) (layer B.Cu) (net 6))
 (segment (start 220.345 86.36) (end 226.06 86.36) (width 0.4) (layer B.Cu) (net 6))
 (segment (start 166.37 80.01) (end 168.275 81.915) (width 0.4) (layer B.Cu) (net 6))
 (segment (start 193.04 81.915) (end 194.31 83.185) (width 0.4) (layer B.Cu) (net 6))
 (segment (start 194.31 83.185) (end 204.47 83.185) (width 0.4) (layer B.Cu) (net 6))
 (segment (start 228.206002 84.213998) (end 228.993998 84.213998) (width 0.4) (layer B.Cu) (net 6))
 (segment (start 230.505 87.045) (end 228.65 88.9) (width 0.4) (layer B.Cu) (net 6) (status 20))
 (segment (start 215.9 88.9) (end 228.6 88.9) (width 0.4) (layer B.Cu) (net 6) (status 30))
 (segment (start 203.2 88.9) (end 215.9 88.9) (width 0.4) (layer B.Cu) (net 6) (status 30))
 (segment (start 190.5 88.9) (end 203.2 88.9) (width 0.4) (layer B.Cu) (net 6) (status 30))
 (segment (start 177.8 88.9) (end 190.5 88.9) (width 0.4) (layer B.Cu) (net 6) (status 30))
 (segment (start 165.1 88.9) (end 177.8 88.9) (width 0.4) (layer B.Cu) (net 6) (status 30))
 (segment (start 152.4 88.9) (end 165.1 88.9) (width 0.4) (layer B.Cu) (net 6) (status 30))
 (segment (start 139.7 88.9) (end 152.4 88.9) (width 0.4) (layer B.Cu) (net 6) (status 30)))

